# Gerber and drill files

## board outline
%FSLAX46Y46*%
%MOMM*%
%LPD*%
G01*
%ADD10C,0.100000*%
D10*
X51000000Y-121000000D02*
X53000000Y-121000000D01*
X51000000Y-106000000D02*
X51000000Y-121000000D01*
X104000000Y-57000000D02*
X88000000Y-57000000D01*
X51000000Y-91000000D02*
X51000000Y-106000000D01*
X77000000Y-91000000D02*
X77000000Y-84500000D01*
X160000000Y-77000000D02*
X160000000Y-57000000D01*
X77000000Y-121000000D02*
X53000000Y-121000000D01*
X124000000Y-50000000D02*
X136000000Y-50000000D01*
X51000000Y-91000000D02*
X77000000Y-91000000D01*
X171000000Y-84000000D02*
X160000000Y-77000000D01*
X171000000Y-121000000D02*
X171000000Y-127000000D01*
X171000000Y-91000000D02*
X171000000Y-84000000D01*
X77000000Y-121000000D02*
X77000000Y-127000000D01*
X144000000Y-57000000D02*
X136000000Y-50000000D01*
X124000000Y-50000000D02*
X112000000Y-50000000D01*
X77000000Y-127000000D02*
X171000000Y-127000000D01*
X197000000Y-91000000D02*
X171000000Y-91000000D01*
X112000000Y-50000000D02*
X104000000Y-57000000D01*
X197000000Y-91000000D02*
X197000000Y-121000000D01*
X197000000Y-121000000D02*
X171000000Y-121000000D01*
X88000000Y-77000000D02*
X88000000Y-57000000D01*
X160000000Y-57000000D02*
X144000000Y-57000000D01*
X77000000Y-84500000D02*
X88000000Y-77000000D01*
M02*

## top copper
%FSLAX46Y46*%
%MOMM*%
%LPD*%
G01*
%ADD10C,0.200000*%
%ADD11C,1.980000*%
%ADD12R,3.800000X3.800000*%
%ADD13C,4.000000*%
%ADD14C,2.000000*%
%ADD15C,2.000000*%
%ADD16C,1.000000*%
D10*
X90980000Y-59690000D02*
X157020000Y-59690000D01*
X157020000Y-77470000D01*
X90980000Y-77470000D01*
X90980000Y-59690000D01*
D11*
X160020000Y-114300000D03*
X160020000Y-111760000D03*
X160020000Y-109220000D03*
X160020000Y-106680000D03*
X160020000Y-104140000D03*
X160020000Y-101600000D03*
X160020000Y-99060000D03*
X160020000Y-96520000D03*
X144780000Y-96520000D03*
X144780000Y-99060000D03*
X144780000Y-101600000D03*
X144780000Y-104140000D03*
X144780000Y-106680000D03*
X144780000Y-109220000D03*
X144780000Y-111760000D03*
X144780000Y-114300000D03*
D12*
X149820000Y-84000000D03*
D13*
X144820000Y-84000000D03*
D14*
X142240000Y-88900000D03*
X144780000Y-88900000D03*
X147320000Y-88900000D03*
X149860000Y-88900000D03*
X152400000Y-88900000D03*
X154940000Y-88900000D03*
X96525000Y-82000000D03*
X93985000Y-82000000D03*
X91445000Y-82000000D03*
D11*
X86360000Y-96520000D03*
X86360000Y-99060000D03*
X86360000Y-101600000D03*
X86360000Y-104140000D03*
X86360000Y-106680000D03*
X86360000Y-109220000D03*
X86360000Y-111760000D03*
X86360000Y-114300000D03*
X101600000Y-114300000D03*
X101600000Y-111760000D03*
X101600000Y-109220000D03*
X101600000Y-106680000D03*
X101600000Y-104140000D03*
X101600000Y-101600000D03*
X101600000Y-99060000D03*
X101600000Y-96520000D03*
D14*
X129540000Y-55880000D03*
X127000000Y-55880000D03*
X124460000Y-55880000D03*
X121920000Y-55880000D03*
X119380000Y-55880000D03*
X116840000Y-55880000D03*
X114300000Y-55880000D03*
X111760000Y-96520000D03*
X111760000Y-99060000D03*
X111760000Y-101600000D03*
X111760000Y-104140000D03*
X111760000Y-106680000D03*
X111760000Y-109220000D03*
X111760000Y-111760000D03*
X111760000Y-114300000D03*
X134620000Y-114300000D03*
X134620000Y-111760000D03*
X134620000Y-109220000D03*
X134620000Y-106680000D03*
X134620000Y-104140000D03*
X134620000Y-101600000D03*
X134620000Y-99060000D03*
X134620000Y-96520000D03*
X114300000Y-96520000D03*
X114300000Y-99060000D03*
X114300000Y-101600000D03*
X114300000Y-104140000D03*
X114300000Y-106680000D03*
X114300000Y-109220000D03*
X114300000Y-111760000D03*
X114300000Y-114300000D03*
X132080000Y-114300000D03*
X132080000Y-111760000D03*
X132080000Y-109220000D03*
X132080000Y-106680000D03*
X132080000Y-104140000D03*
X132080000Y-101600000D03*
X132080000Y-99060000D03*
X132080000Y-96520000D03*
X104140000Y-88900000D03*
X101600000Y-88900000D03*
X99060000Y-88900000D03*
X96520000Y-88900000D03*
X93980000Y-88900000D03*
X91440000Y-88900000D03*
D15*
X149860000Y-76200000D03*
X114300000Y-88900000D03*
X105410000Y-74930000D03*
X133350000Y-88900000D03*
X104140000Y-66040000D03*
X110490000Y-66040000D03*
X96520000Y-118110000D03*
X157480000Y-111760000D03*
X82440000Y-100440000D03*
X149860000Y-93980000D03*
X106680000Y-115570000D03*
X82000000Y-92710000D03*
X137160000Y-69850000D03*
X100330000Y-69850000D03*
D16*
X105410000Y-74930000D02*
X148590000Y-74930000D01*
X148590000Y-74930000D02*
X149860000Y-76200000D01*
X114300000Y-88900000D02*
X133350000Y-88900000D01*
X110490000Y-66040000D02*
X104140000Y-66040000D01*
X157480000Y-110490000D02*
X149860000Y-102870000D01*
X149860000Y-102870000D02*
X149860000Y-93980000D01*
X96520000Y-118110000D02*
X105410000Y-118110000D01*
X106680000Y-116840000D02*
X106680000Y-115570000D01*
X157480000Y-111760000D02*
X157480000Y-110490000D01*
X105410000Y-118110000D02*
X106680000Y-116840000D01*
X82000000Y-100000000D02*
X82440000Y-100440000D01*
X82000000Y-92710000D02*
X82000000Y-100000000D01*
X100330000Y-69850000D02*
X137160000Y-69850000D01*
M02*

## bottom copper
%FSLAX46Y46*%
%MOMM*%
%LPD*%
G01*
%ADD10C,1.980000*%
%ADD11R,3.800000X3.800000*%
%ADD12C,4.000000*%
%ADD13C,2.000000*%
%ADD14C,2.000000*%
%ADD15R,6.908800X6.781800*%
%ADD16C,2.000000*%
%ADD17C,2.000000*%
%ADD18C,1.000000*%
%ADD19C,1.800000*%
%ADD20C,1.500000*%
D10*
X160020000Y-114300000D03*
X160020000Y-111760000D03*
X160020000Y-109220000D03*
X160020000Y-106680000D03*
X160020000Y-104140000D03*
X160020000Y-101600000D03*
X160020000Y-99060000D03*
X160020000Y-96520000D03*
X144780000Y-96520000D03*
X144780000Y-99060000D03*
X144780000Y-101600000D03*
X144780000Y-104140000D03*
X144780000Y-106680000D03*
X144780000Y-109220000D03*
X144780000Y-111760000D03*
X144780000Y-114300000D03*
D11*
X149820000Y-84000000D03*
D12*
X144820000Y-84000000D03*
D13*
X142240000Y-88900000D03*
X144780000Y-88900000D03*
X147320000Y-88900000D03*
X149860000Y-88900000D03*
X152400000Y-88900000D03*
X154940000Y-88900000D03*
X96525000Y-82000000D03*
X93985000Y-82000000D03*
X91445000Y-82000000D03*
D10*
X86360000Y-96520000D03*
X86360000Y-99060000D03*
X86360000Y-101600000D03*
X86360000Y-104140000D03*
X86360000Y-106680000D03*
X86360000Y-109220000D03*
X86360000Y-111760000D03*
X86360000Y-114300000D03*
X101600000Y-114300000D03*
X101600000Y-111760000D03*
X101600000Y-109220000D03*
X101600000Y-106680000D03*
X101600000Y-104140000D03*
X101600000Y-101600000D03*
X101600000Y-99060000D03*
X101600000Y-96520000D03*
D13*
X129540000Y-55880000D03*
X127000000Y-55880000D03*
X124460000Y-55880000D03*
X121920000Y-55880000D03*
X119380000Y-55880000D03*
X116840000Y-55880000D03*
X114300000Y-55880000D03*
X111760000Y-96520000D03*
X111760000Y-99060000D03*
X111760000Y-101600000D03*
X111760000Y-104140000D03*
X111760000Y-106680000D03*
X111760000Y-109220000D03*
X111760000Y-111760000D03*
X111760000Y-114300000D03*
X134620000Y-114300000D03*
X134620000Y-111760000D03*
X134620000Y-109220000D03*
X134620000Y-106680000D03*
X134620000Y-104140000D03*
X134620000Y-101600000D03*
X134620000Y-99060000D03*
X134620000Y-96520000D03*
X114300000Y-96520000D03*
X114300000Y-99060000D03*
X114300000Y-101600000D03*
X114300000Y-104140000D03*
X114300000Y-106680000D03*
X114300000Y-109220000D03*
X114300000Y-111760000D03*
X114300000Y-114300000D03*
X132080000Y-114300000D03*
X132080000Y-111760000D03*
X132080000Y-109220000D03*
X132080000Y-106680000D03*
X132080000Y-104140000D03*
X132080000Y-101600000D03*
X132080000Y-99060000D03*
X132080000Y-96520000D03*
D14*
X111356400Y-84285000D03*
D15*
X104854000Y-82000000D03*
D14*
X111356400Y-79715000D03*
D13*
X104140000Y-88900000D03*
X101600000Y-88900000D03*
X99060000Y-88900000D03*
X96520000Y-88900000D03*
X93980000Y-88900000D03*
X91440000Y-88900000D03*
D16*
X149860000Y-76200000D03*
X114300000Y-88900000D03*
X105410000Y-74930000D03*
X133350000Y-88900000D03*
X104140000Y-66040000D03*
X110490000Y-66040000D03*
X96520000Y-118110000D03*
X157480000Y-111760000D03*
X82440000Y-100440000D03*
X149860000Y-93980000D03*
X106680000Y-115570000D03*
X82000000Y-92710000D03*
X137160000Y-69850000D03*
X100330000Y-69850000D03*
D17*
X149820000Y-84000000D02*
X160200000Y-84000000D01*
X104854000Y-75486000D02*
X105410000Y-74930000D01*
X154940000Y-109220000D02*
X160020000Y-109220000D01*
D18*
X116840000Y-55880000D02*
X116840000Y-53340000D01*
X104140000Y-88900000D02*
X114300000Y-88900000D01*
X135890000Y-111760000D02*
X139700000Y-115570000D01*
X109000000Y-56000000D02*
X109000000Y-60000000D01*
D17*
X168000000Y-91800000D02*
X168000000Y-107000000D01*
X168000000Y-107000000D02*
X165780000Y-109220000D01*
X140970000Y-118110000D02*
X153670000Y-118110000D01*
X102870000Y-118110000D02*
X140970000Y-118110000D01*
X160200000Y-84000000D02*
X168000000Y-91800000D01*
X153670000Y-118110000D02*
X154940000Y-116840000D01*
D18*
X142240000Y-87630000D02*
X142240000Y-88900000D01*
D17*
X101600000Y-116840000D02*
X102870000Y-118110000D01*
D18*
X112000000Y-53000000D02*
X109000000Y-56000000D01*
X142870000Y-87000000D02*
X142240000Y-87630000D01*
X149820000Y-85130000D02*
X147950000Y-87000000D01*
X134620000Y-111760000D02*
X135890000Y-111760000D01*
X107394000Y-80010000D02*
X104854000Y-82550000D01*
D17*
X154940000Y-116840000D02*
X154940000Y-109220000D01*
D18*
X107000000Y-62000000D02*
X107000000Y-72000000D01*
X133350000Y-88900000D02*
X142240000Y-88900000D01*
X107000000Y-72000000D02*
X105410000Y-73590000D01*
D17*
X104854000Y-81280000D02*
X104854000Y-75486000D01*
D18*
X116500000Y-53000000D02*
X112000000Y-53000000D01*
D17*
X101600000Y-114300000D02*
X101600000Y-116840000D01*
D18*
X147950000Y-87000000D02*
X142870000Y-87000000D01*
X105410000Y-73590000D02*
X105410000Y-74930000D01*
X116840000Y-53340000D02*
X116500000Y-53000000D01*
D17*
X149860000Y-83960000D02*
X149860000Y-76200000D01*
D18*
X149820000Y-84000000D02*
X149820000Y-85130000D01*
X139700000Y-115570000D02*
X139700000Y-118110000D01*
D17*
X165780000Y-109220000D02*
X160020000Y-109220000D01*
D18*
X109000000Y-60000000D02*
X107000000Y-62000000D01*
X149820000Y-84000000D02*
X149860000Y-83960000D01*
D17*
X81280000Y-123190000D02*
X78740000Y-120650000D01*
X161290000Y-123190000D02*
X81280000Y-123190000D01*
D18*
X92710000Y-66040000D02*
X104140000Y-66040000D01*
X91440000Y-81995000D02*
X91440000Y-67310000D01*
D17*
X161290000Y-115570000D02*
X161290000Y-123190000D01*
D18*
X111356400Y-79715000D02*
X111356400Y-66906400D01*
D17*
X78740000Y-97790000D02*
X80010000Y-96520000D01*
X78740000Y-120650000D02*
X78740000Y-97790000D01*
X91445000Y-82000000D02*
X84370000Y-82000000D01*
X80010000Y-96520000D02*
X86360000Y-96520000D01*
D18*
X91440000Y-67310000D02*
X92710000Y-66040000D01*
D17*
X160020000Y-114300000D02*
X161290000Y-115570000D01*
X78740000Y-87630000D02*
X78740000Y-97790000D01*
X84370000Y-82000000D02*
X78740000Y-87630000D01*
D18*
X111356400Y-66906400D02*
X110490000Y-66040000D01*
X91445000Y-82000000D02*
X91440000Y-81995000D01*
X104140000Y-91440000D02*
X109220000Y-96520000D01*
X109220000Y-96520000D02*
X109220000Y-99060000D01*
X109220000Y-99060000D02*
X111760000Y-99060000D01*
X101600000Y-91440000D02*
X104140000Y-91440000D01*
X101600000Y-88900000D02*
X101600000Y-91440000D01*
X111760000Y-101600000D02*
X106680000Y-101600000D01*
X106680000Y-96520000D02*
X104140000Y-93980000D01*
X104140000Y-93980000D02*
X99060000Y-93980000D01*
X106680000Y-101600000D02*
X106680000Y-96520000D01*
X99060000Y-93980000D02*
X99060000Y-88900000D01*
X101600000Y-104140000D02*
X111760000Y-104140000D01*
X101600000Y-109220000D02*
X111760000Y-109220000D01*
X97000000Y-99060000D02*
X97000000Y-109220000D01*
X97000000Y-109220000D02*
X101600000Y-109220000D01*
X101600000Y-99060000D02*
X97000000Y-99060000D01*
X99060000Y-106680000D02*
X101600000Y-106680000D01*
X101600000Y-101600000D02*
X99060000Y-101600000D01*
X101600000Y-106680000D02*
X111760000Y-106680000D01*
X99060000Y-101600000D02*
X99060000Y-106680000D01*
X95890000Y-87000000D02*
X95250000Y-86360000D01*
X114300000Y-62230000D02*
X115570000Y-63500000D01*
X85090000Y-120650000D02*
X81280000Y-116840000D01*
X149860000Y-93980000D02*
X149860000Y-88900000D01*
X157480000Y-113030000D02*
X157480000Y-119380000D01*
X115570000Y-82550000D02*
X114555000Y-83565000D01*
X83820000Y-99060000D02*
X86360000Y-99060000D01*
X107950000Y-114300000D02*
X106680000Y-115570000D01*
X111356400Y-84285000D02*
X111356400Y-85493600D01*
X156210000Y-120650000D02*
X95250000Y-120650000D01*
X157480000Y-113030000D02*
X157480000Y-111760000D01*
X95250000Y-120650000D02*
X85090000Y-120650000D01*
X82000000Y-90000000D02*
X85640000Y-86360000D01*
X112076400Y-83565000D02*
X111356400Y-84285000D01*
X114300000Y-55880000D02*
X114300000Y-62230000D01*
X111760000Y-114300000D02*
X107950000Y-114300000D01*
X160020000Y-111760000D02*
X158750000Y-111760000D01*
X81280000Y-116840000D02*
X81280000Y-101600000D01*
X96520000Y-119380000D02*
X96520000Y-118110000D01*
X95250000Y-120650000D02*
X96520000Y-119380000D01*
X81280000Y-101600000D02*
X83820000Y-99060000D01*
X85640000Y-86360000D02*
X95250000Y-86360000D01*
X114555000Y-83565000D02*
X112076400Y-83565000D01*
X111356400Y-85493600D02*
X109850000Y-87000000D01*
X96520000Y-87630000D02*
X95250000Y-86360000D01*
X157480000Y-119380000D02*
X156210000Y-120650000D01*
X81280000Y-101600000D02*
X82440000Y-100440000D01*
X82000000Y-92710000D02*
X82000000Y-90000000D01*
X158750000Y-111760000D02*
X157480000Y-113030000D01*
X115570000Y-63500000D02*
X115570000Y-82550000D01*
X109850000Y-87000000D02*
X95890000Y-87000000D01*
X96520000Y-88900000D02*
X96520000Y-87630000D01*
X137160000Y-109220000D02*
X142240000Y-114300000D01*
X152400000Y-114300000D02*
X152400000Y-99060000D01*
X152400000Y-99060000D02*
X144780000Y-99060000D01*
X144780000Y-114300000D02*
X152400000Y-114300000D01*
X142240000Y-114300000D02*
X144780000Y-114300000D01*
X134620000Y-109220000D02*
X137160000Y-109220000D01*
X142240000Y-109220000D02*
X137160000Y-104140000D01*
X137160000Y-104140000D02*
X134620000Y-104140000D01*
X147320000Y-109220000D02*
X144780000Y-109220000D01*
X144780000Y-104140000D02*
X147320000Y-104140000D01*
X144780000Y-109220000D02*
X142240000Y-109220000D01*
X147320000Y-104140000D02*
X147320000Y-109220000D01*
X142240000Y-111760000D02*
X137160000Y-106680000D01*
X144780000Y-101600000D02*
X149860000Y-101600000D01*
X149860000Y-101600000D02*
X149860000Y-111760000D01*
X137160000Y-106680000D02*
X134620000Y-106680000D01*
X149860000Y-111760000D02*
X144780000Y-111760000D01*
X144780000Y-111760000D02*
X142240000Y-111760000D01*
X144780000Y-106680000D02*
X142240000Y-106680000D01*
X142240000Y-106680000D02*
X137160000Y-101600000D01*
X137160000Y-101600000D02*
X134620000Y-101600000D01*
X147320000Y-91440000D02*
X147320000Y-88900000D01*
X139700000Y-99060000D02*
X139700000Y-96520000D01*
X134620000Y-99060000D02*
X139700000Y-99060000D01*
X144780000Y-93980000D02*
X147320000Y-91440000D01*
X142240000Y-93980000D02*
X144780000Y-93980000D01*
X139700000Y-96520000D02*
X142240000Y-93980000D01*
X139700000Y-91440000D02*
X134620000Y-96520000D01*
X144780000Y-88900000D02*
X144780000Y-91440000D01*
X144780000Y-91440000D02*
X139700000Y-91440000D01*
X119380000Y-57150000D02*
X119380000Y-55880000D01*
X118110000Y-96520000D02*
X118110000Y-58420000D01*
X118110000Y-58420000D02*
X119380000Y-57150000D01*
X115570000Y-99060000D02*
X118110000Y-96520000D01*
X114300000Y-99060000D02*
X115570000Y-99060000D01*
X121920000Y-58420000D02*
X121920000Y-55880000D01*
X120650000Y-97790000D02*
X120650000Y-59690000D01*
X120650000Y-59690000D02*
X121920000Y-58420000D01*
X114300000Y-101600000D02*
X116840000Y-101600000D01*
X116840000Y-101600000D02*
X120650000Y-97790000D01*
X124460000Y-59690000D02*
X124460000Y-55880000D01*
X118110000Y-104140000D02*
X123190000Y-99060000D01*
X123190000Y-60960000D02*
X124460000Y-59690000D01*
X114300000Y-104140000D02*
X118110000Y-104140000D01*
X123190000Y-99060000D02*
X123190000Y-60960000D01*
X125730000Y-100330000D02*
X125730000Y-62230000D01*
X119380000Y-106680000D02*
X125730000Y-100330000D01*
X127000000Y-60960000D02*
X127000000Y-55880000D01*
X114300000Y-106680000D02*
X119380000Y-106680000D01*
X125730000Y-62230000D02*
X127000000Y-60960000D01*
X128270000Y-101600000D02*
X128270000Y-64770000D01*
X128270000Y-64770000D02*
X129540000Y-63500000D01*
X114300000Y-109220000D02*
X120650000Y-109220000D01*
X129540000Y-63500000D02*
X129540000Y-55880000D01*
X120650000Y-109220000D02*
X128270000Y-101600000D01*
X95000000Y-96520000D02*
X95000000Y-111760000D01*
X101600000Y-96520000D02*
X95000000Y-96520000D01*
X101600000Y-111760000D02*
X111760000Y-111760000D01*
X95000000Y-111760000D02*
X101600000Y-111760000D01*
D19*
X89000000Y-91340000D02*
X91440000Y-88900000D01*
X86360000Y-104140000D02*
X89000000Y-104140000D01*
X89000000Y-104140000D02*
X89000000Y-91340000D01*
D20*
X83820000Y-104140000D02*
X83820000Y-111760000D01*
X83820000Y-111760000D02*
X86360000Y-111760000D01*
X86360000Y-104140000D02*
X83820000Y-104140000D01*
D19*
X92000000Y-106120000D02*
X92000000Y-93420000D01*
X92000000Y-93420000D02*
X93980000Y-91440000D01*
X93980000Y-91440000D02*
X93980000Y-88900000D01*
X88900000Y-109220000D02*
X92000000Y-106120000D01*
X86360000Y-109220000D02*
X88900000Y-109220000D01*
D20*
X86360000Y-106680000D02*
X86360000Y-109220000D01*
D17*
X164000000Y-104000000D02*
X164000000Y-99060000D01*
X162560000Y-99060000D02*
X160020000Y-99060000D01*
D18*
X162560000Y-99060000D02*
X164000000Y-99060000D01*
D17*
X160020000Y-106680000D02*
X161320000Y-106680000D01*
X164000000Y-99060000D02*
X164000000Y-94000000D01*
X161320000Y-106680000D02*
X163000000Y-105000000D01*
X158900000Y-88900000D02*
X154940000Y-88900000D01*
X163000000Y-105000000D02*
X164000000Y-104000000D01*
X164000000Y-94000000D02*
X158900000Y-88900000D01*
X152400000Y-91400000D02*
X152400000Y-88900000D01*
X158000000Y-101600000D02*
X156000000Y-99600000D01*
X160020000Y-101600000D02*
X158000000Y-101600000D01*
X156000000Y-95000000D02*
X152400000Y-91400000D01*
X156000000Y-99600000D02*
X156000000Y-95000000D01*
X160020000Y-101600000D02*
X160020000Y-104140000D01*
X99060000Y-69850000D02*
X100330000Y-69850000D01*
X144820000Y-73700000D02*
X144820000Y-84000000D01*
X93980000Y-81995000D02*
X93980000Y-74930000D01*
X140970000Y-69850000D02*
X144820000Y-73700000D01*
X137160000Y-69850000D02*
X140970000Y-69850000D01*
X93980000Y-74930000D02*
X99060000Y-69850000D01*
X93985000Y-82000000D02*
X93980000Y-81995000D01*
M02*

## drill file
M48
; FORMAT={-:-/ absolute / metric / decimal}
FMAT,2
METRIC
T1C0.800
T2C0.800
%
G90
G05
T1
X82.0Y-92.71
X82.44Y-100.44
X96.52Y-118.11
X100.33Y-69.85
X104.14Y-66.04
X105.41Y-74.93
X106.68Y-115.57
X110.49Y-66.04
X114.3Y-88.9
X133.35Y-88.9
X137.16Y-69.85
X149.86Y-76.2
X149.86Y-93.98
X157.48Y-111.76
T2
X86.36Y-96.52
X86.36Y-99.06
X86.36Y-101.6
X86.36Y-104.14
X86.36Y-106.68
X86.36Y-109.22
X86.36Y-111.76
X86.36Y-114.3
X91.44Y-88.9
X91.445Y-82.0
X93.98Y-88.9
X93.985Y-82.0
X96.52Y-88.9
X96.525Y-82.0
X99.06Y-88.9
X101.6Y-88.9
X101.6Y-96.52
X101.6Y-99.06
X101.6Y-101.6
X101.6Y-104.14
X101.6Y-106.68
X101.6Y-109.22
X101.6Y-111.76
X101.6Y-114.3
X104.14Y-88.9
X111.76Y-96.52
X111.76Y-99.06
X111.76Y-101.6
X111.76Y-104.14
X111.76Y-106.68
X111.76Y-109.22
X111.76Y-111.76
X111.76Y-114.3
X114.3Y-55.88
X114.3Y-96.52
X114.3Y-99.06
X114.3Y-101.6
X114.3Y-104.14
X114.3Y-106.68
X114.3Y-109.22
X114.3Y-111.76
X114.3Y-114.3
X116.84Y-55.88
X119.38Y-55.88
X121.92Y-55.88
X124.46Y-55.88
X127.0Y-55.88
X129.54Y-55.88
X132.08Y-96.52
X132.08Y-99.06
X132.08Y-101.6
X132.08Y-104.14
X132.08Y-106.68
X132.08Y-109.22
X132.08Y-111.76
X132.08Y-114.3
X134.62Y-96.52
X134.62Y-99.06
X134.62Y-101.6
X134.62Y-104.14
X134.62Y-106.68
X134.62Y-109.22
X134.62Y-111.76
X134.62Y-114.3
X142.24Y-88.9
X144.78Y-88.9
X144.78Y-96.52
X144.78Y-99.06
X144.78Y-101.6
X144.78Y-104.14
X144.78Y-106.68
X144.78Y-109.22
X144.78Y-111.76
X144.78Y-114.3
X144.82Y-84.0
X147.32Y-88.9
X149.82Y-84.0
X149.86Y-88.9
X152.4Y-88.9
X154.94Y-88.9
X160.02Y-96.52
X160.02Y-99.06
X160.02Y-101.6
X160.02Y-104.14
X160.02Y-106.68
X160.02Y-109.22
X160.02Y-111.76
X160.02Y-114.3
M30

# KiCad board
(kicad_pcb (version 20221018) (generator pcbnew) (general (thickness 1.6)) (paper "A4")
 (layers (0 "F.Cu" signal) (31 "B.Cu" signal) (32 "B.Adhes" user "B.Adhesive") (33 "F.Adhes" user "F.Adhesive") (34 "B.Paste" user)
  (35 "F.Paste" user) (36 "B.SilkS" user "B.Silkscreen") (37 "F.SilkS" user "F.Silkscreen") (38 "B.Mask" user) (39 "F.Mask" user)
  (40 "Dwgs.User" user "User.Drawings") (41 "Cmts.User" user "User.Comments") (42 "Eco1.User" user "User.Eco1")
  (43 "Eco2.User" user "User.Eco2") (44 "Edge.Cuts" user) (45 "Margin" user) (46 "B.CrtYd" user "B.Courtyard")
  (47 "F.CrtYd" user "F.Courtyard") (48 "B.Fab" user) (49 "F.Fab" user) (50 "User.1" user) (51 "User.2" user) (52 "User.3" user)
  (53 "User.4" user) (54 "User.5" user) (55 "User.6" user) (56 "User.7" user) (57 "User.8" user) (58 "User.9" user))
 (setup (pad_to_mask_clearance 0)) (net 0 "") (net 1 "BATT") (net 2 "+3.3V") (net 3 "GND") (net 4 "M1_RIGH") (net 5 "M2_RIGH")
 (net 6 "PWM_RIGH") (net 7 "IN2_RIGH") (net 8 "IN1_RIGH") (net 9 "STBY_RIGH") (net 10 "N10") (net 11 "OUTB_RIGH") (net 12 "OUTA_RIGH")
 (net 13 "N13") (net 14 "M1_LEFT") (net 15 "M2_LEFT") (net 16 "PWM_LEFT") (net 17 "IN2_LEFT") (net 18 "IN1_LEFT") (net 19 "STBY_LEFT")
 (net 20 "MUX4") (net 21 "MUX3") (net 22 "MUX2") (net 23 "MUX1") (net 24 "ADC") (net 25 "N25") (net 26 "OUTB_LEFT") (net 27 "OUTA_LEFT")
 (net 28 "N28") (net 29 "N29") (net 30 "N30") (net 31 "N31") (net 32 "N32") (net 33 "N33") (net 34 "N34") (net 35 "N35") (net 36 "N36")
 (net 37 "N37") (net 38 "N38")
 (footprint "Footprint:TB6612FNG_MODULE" (layer "F.Cu") (at 152.4 105.41 180)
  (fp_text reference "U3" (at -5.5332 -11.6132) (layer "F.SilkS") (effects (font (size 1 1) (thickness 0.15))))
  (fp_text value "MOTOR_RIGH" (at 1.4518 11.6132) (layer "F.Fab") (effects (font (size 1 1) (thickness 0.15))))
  (pad "1" thru_hole circle (at -7.62 -8.89 180) (size 1.98 1.98) (drill 0.8) (layers "*.Cu" "*.Mask") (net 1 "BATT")
   (solder_mask_margin 0.102))
  (pad "2" thru_hole circle (at -7.62 -6.35 180) (size 1.98 1.98) (drill 0.8) (layers "*.Cu" "*.Mask") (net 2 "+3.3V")
   (solder_mask_margin 0.102))
  (pad "3" thru_hole circle (at -7.62 -3.81 180) (size 1.98 1.98) (drill 0.8) (layers "*.Cu" "*.Mask") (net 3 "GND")
   (solder_mask_margin 0.102))
  (pad "4" thru_hole circle (at -7.62 -1.27 180) (size 1.98 1.98) (drill 0.8) (layers "*.Cu" "*.Mask") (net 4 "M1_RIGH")
   (solder_mask_margin 0.102))
  (pad "5" thru_hole circle (at -7.62 1.27 180) (size 1.98 1.98) (drill 0.8) (layers "*.Cu" "*.Mask") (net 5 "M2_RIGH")
   (solder_mask_margin 0.102))
  (pad "6" thru_hole circle (at -7.62 3.81 180) (size 1.98 1.98) (drill 0.8) (layers "*.Cu" "*.Mask") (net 5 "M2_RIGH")
   (solder_mask_margin 0.102))
  (pad "7" thru_hole circle (at -7.62 6.35 180) (size 1.98 1.98) (drill 0.8) (layers "*.Cu" "*.Mask") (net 4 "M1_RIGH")
   (solder_mask_margin 0.102))
  (pad "8" thru_hole circle (at -7.62 8.89 180) (size 1.98 1.98) (drill 0.8) (layers "*.Cu" "*.Mask") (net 3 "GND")
   (solder_mask_margin 0.102))
  (pad "9" thru_hole circle (at 7.62 8.89 180) (size 1.98 1.98) (drill 0.8) (layers "*.Cu" "*.Mask") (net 3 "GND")
   (solder_mask_margin 0.102))
  (pad "10" thru_hole circle (at 7.62 6.35 180) (size 1.98 1.98) (drill 0.8) (layers "*.Cu" "*.Mask") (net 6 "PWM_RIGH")
   (solder_mask_margin 0.102))
  (pad "11" thru_hole circle (at 7.62 3.81 180) (size 1.98 1.98) (drill 0.8) (layers "*.Cu" "*.Mask") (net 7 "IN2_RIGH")
   (solder_mask_margin 0.102))
  (pad "12" thru_hole circle (at 7.62 1.27 180) (size 1.98 1.98) (drill 0.8) (layers "*.Cu" "*.Mask") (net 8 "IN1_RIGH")
   (solder_mask_margin 0.102))
  (pad "13" thru_hole circle (at 7.62 -1.27 180) (size 1.98 1.98) (drill 0.8) (layers "*.Cu" "*.Mask") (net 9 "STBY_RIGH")
   (solder_mask_margin 0.102))
  (pad "14" thru_hole circle (at 7.62 -3.81 180) (size 1.98 1.98) (drill 0.8) (layers "*.Cu" "*.Mask") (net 8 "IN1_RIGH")
   (solder_mask_margin 0.102))
  (pad "15" thru_hole circle (at 7.62 -6.35 180) (size 1.98 1.98) (drill 0.8) (layers "*.Cu" "*.Mask") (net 7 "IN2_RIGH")
   (solder_mask_margin 0.102))
  (pad "16" thru_hole circle (at 7.62 -8.89 180) (size 1.98 1.98) (drill 0.8) (layers "*.Cu" "*.Mask") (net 6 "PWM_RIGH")
   (solder_mask_margin 0.102)))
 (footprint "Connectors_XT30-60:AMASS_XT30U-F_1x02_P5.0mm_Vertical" (layer "F.Cu") (at 149.82 84 180)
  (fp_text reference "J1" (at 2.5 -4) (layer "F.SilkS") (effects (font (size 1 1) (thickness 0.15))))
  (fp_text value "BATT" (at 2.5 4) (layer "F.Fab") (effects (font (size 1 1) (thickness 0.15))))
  (pad "1" thru_hole rect (at 0 0 180) (size 3.8 3.8) (drill 0.8) (layers "*.Cu" "*.Mask") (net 3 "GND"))
  (pad "2" thru_hole circle (at 5 0 180) (size 4 4) (drill 0.8) (layers "*.Cu" "*.Mask") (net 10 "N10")))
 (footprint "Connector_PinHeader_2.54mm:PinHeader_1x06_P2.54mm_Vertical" (layer "F.Cu") (at 142.24 88.9 90)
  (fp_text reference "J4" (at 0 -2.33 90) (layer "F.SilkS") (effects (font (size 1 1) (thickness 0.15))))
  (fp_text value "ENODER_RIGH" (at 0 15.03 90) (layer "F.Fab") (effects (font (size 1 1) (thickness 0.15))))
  (pad "1" thru_hole circle (at 0 0 90) (size 2 2) (drill 0.8) (layers "*.Cu" "*.Mask") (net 3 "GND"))
  (pad "2" thru_hole circle (at 0 2.54 90) (size 2 2) (drill 0.8) (layers "*.Cu" "*.Mask") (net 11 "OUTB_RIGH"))
  (pad "3" thru_hole circle (at 0 5.08 90) (size 2 2) (drill 0.8) (layers "*.Cu" "*.Mask") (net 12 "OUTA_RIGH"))
  (pad "4" thru_hole circle (at 0 7.62 90) (size 2 2) (drill 0.8) (layers "*.Cu" "*.Mask") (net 2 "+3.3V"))
  (pad "5" thru_hole circle (at 0 10.16 90) (size 2 2) (drill 0.8) (layers "*.Cu" "*.Mask") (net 5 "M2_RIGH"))
  (pad "6" thru_hole circle (at 0 12.7 90) (size 2 2) (drill 0.8) (layers "*.Cu" "*.Mask") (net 4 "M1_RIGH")))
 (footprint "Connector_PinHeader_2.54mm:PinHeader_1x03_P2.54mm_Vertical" (layer "F.Cu") (at 96.525 82 -90)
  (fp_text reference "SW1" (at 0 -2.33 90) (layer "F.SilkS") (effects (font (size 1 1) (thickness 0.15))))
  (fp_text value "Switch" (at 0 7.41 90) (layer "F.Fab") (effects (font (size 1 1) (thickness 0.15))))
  (pad "1" thru_hole circle (at 0 0 270) (size 2 2) (drill 0.8) (layers "*.Cu" "*.Mask") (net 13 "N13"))
  (pad "2" thru_hole circle (at 0 2.54 270) (size 2 2) (drill 0.8) (layers "*.Cu" "*.Mask") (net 10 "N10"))
  (pad "3" thru_hole circle (at 0 5.08 270) (size 2 2) (drill 0.8) (layers "*.Cu" "*.Mask") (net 1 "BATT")))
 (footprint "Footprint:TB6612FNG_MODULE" (layer "F.Cu") (at 93.98 105.41)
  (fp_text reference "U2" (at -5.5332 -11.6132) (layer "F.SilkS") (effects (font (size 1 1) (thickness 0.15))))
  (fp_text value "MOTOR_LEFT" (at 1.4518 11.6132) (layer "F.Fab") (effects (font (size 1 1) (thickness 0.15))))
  (pad "1" thru_hole circle (at -7.62 -8.89) (size 1.98 1.98) (drill 0.8) (layers "*.Cu" "*.Mask") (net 1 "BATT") (solder_mask_margin 0.102))
  (pad "2" thru_hole circle (at -7.62 -6.35) (size 1.98 1.98) (drill 0.8) (layers "*.Cu" "*.Mask") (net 2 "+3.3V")
   (solder_mask_margin 0.102))
  (pad "3" thru_hole circle (at -7.62 -3.81) (size 1.98 1.98) (drill 0.8) (layers "*.Cu" "*.Mask") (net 3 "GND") (solder_mask_margin 0.102))
  (pad "4" thru_hole circle (at -7.62 -1.27) (size 1.98 1.98) (drill 0.8) (layers "*.Cu" "*.Mask") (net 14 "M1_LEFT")
   (solder_mask_margin 0.102))
  (pad "5" thru_hole circle (at -7.62 1.27) (size 1.98 1.98) (drill 0.8) (layers "*.Cu" "*.Mask") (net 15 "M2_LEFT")
   (solder_mask_margin 0.102))
  (pad "6" thru_hole circle (at -7.62 3.81) (size 1.98 1.98) (drill 0.8) (layers "*.Cu" "*.Mask") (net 15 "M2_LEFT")
   (solder_mask_margin 0.102))
  (pad "7" thru_hole circle (at -7.62 6.35) (size 1.98 1.98) (drill 0.8) (layers "*.Cu" "*.Mask") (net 14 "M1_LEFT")
   (solder_mask_margin 0.102))
  (pad "8" thru_hole circle (at -7.62 8.89) (size 1.98 1.98) (drill 0.8) (layers "*.Cu" "*.Mask") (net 3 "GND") (solder_mask_margin 0.102))
  (pad "9" thru_hole circle (at 7.62 8.89) (size 1.98 1.98) (drill 0.8) (layers "*.Cu" "*.Mask") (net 3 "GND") (solder_mask_margin 0.102))
  (pad "10" thru_hole circle (at 7.62 6.35) (size 1.98 1.98) (drill 0.8) (layers "*.Cu" "*.Mask") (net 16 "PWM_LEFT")
   (solder_mask_margin 0.102))
  (pad "11" thru_hole circle (at 7.62 3.81) (size 1.98 1.98) (drill 0.8) (layers "*.Cu" "*.Mask") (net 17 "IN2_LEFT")
   (solder_mask_margin 0.102))
  (pad "12" thru_hole circle (at 7.62 1.27) (size 1.98 1.98) (drill 0.8) (layers "*.Cu" "*.Mask") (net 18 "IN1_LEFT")
   (solder_mask_margin 0.102))
  (pad "13" thru_hole circle (at 7.62 -1.27) (size 1.98 1.98) (drill 0.8) (layers "*.Cu" "*.Mask") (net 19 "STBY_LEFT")
   (solder_mask_margin 0.102))
  (pad "14" thru_hole circle (at 7.62 -3.81) (size 1.98 1.98) (drill 0.8) (layers "*.Cu" "*.Mask") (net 18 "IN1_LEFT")
   (solder_mask_margin 0.102))
  (pad "15" thru_hole circle (at 7.62 -6.35) (size 1.98 1.98) (drill 0.8) (layers "*.Cu" "*.Mask") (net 17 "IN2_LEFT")
   (solder_mask_margin 0.102))
  (pad "16" thru_hole circle (at 7.62 -8.89) (size 1.98 1.98) (drill 0.8) (layers "*.Cu" "*.Mask") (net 16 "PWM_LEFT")
   (solder_mask_margin 0.102)))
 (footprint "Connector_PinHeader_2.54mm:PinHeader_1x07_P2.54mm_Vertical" (layer "F.Cu") (at 129.54 55.88 -90)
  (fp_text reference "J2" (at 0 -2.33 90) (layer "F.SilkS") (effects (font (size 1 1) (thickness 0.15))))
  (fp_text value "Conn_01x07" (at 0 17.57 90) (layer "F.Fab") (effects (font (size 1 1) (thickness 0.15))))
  (pad "1" thru_hole circle (at 0 0 270) (size 2 2) (drill 0.8) (layers "*.Cu" "*.Mask") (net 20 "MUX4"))
  (pad "2" thru_hole circle (at 0 2.54 270) (size 2 2) (drill 0.8) (layers "*.Cu" "*.Mask") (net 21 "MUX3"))
  (pad "3" thru_hole circle (at 0 5.08 270) (size 2 2) (drill 0.8) (layers "*.Cu" "*.Mask") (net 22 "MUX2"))
  (pad "4" thru_hole circle (at 0 7.62 270) (size 2 2) (drill 0.8) (layers "*.Cu" "*.Mask") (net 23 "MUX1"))
  (pad "5" thru_hole circle (at 0 10.16 270) (size 2 2) (drill 0.8) (layers "*.Cu" "*.Mask") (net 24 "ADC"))
  (pad "6" thru_hole circle (at 0 12.7 270) (size 2 2) (drill 0.8) (layers "*.Cu" "*.Mask") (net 3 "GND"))
  (pad "7" thru_hole circle (at 0 15.24 270) (size 2 2) (drill 0.8) (layers "*.Cu" "*.Mask") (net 2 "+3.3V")))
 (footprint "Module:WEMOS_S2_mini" (layer "F.Cu") (at 111.76 96.52)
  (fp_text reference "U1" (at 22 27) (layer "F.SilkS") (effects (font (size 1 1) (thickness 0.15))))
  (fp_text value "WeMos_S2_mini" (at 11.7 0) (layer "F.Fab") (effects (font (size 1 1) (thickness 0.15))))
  (pad "1" thru_hole circle (at 0 0) (size 2 2) (drill 0.8) (layers "*.Cu" "*.Mask") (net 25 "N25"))
  (pad "2" thru_hole circle (at 0 2.54) (size 2 2) (drill 0.8) (layers "*.Cu" "*.Mask") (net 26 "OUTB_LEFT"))
  (pad "3" thru_hole circle (at 0 5.08) (size 2 2) (drill 0.8) (layers "*.Cu" "*.Mask") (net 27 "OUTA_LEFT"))
  (pad "4" thru_hole circle (at 0 7.62) (size 2 2) (drill 0.8) (layers "*.Cu" "*.Mask") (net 19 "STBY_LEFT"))
  (pad "5" thru_hole circle (at 0 10.16) (size 2 2) (drill 0.8) (layers "*.Cu" "*.Mask") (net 18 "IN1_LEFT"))
  (pad "6" thru_hole circle (at 0 12.7) (size 2 2) (drill 0.8) (layers "*.Cu" "*.Mask") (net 17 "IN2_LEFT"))
  (pad "7" thru_hole circle (at 0 15.24) (size 2 2) (drill 0.8) (layers "*.Cu" "*.Mask") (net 16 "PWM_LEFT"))
  (pad "8" thru_hole circle (at 0 17.78) (size 2 2) (drill 0.8) (layers "*.Cu" "*.Mask") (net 2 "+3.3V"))
  (pad "9" thru_hole circle (at 22.86 17.78) (size 2 2) (drill 0.8) (layers "*.Cu" "*.Mask") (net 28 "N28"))
  (pad "10" thru_hole circle (at 22.86 15.24) (size 2 2) (drill 0.8) (layers "*.Cu" "*.Mask") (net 3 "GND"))
  (pad "11" thru_hole circle (at 22.86 12.7) (size 2 2) (drill 0.8) (layers "*.Cu" "*.Mask") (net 6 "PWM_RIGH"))
  (pad "12" thru_hole circle (at 22.86 10.16) (size 2 2) (drill 0.8) (layers "*.Cu" "*.Mask") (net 7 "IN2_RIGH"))
  (pad "13" thru_hole circle (at 22.86 7.62) (size 2 2) (drill 0.8) (layers "*.Cu" "*.Mask") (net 8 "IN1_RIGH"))
  (pad "14" thru_hole circle (at 22.86 5.08) (size 2 2) (drill 0.8) (layers "*.Cu" "*.Mask") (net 9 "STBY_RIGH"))
  (pad "15" thru_hole circle (at 22.86 2.54) (size 2 2) (drill 0.8) (layers "*.Cu" "*.Mask") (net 12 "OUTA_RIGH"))
  (pad "16" thru_hole circle (at 22.86 0) (size 2 2) (drill 0.8) (layers "*.Cu" "*.Mask") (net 11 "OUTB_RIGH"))
  (pad "17" thru_hole circle (at 2.54 0) (size 2 2) (drill 0.8) (layers "*.Cu" "*.Mask") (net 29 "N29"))
  (pad "18" thru_hole circle (at 2.54 2.54) (size 2 2) (drill 0.8) (layers "*.Cu" "*.Mask") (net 24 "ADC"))
  (pad "19" thru_hole circle (at 2.54 5.08) (size 2 2) (drill 0.8) (layers "*.Cu" "*.Mask") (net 23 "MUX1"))
  (pad "20" thru_hole circle (at 2.54 7.62) (size 2 2) (drill 0.8) (layers "*.Cu" "*.Mask") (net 22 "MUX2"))
  (pad "21" thru_hole circle (at 2.54 10.16) (size 2 2) (drill 0.8) (layers "*.Cu" "*.Mask") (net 21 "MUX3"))
  (pad "22" thru_hole circle (at 2.54 12.7) (size 2 2) (drill 0.8) (layers "*.Cu" "*.Mask") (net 20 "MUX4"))
  (pad "23" thru_hole circle (at 2.54 15.24) (size 2 2) (drill 0.8) (layers "*.Cu" "*.Mask") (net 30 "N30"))
  (pad "24" thru_hole circle (at 2.54 17.78) (size 2 2) (drill 0.8) (layers "*.Cu" "*.Mask") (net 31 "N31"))
  (pad "25" thru_hole circle (at 20.32 17.78) (size 2 2) (drill 0.8) (layers "*.Cu" "*.Mask") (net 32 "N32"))
  (pad "26" thru_hole circle (at 20.32 15.24) (size 2 2) (drill 0.8) (layers "*.Cu" "*.Mask") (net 3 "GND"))
  (pad "27" thru_hole circle (at 20.32 12.7) (size 2 2) (drill 0.8) (layers "*.Cu" "*.Mask") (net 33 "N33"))
  (pad "28" thru_hole circle (at 20.32 10.16) (size 2 2) (drill 0.8) (layers "*.Cu" "*.Mask") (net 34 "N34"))
  (pad "29" thru_hole circle (at 20.32 7.62) (size 2 2) (drill 0.8) (layers "*.Cu" "*.Mask") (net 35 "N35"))
  (pad "30" thru_hole circle (at 20.32 5.08) (size 2 2) (drill 0.8) (layers "*.Cu" "*.Mask") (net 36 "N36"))
  (pad "31" thru_hole circle (at 20.32 2.54) (size 2 2) (drill 0.8) (layers "*.Cu" "*.Mask") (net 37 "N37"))
  (pad "32" thru_hole circle (at 20.32 0) (size 2 2) (drill 0.8) (layers "*.Cu" "*.Mask") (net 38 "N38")))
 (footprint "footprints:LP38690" (layer "F.Cu") (at 104.854 82 90)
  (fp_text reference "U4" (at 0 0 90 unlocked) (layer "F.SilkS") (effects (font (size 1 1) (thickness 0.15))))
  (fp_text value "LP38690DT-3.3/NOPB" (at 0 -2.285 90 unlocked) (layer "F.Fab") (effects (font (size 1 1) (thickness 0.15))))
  (pad "1" smd circle (at -2.285 6.5024 90) (size 2 2) (layers "B.Cu" "F.Paste" "F.Mask") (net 2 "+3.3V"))
  (pad "2" smd rect (at 0 0 90) (size 6.7818 6.9088) (layers "B.Cu" "F.Paste" "F.Mask") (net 3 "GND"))
  (pad "3" smd circle (at 2.285 6.5024 90) (size 2 2) (layers "B.Cu" "F.Paste" "F.Mask") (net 1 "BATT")))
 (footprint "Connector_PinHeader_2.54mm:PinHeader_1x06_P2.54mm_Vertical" (layer "F.Cu") (at 104.14 88.9 -90)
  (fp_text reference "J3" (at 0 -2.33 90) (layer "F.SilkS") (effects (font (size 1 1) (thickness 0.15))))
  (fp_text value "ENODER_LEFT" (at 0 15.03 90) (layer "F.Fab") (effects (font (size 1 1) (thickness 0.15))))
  (pad "1" thru_hole circle (at 0 0 270) (size 2 2) (drill 0.8) (layers "*.Cu" "*.Mask") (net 3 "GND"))
  (pad "2" thru_hole circle (at 0 2.54 270) (size 2 2) (drill 0.8) (layers "*.Cu" "*.Mask") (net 26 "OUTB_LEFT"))
  (pad "3" thru_hole circle (at 0 5.08 270) (size 2 2) (drill 0.8) (layers "*.Cu" "*.Mask") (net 27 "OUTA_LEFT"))
  (pad "4" thru_hole circle (at 0 7.62 270) (size 2 2) (drill 0.8) (layers "*.Cu" "*.Mask") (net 2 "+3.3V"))
  (pad "5" thru_hole circle (at 0 10.16 270) (size 2 2) (drill 0.8) (layers "*.Cu" "*.Mask") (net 15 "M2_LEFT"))
  (pad "6" thru_hole circle (at 0 12.7 270) (size 2 2) (drill 0.8) (layers "*.Cu" "*.Mask") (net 14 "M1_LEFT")))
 (gr_rect (start 90.98 59.69) (end 157.02 77.47) (stroke (width 0.2) (type default)) (fill none) (layer "F.Cu"))
 (gr_line (start 51 121) (end 53 121) (stroke (width 0.1) (type default)) (layer "Edge.Cuts"))
 (gr_line (start 51 106) (end 51 121) (stroke (width 0.1) (type default)) (layer "Edge.Cuts"))
 (gr_line (start 104 57) (end 88 57) (stroke (width 0.1) (type default)) (layer "Edge.Cuts"))
 (gr_line (start 51 91) (end 51 106) (stroke (width 0.1) (type default)) (layer "Edge.Cuts"))
 (gr_line (start 77 91) (end 77 84.5) (stroke (width 0.1) (type default)) (layer "Edge.Cuts"))
 (gr_line (start 160 77) (end 160 57) (stroke (width 0.1) (type default)) (layer "Edge.Cuts"))
 (gr_line (start 77 121) (end 53 121) (stroke (width 0.1) (type default)) (layer "Edge.Cuts"))
 (gr_line (start 124 50) (end 136 50) (stroke (width 0.1) (type default)) (layer "Edge.Cuts"))
 (gr_line (start 51 91) (end 77 91) (stroke (width 0.1) (type default)) (layer "Edge.Cuts"))
 (gr_line (start 171 84) (end 160 77) (stroke (width 0.1) (type default)) (layer "Edge.Cuts"))
 (gr_line (start 171 121) (end 171 127) (stroke (width 0.1) (type default)) (layer "Edge.Cuts"))
 (gr_line (start 171 91) (end 171 84) (stroke (width 0.1) (type default)) (layer "Edge.Cuts"))
 (gr_line (start 77 121) (end 77 127) (stroke (width 0.1) (type default)) (layer "Edge.Cuts"))
 (gr_line (start 144 57) (end 136 50) (stroke (width 0.1) (type default)) (layer "Edge.Cuts"))
 (gr_line (start 124 50) (end 112 50) (stroke (width 0.1) (type default)) (layer "Edge.Cuts"))
 (gr_line (start 77 127) (end 171 127) (stroke (width 0.1) (type default)) (layer "Edge.Cuts"))
 (gr_line (start 197 91) (end 171 91) (stroke (width 0.1) (type default)) (layer "Edge.Cuts"))
 (gr_line (start 112 50) (end 104 57) (stroke (width 0.1) (type default)) (layer "Edge.Cuts"))
 (gr_line (start 197 91) (end 197 121) (stroke (width 0.1) (type default)) (layer "Edge.Cuts"))
 (gr_line (start 197 121) (end 171 121) (stroke (width 0.1) (type default)) (layer "Edge.Cuts"))
 (gr_line (start 88 77) (end 88 57) (stroke (width 0.1) (type default)) (layer "Edge.Cuts"))
 (gr_line (start 160 57) (end 144 57) (stroke (width 0.1) (type default)) (layer "Edge.Cuts"))
 (gr_line (start 77 84.5) (end 88 77) (stroke (width 0.1) (type default)) (layer "Edge.Cuts"))
 (segment (start 105.41 74.93) (end 148.59 74.93) (width 1) (layer "F.Cu") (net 3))
 (segment (start 148.59 74.93) (end 149.86 76.2) (width 1) (layer "F.Cu") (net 3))
 (segment (start 114.3 88.9) (end 133.35 88.9) (width 1) (layer "F.Cu") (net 3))
 (via (at 149.86 76.2) (size 2) (drill 0.8) (layers "F.Cu" "B.Cu") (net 3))
 (via (at 114.3 88.9) (size 2) (drill 0.8) (layers "F.Cu" "B.Cu") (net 3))
 (via (at 105.41 74.93) (size 2) (drill 0.8) (layers "F.Cu" "B.Cu") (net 3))
 (via (at 133.35 88.9) (size 2) (drill 0.8) (layers "F.Cu" "B.Cu") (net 3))
 (segment (start 149.82 84) (end 160.2 84) (width 2) (layer "B.Cu") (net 3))
 (segment (start 104.854 75.486) (end 105.41 74.93) (width 2) (layer "B.Cu") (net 3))
 (segment (start 154.94 109.22) (end 160.02 109.22) (width 2) (layer "B.Cu") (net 3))
 (segment (start 116.84 55.88) (end 116.84 53.34) (width 1) (layer "B.Cu") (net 3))
 (segment (start 104.14 88.9) (end 114.3 88.9) (width 1) (layer "B.Cu") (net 3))
 (segment (start 135.89 111.76) (end 139.7 115.57) (width 1) (layer "B.Cu") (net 3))
 (segment (start 109 56) (end 109 60) (width 1) (layer "B.Cu") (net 3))
 (segment (start 168 91.8) (end 168 107) (width 2) (layer "B.Cu") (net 3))
 (segment (start 168 107) (end 165.78 109.22) (width 2) (layer "B.Cu") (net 3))
 (segment (start 140.97 118.11) (end 153.67 118.11) (width 2) (layer "B.Cu") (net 3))
 (segment (start 102.87 118.11) (end 140.97 118.11) (width 2) (layer "B.Cu") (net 3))
 (segment (start 160.2 84) (end 168 91.8) (width 2) (layer "B.Cu") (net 3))
 (segment (start 153.67 118.11) (end 154.94 116.84) (width 2) (layer "B.Cu") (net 3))
 (segment (start 142.24 87.63) (end 142.24 88.9) (width 1) (layer "B.Cu") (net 3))
 (segment (start 101.6 116.84) (end 102.87 118.11) (width 2) (layer "B.Cu") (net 3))
 (segment (start 112 53) (end 109 56) (width 1) (layer "B.Cu") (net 3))
 (segment (start 142.87 87) (end 142.24 87.63) (width 1) (layer "B.Cu") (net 3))
 (segment (start 149.82 85.13) (end 147.95 87) (width 1) (layer "B.Cu") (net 3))
 (segment (start 134.62 111.76) (end 135.89 111.76) (width 1) (layer "B.Cu") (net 3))
 (segment (start 107.394 80.01) (end 104.854 82.55) (width 1) (layer "B.Cu") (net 3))
 (segment (start 154.94 116.84) (end 154.94 109.22) (width 2) (layer "B.Cu") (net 3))
 (segment (start 107 62) (end 107 72) (width 1) (layer "B.Cu") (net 3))
 (segment (start 133.35 88.9) (end 142.24 88.9) (width 1) (layer "B.Cu") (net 3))
 (segment (start 107 72) (end 105.41 73.59) (width 1) (layer "B.Cu") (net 3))
 (segment (start 104.854 81.28) (end 104.854 75.486) (width 2) (layer "B.Cu") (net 3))
 (segment (start 116.5 53) (end 112 53) (width 1) (layer "B.Cu") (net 3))
 (segment (start 101.6 114.3) (end 101.6 116.84) (width 2) (layer "B.Cu") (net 3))
 (segment (start 147.95 87) (end 142.87 87) (width 1) (layer "B.Cu") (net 3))
 (segment (start 105.41 73.59) (end 105.41 74.93) (width 1) (layer "B.Cu") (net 3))
 (segment (start 116.84 53.34) (end 116.5 53) (width 1) (layer "B.Cu") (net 3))
 (segment (start 149.86 83.96) (end 149.86 76.2) (width 2) (layer "B.Cu") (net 3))
 (segment (start 149.82 84) (end 149.82 85.13) (width 1) (layer "B.Cu") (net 3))
 (segment (start 139.7 115.57) (end 139.7 118.11) (width 1) (layer "B.Cu") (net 3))
 (segment (start 165.78 109.22) (end 160.02 109.22) (width 2) (layer "B.Cu") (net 3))
 (segment (start 109 60) (end 107 62) (width 1) (layer "B.Cu") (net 3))
 (segment (start 149.82 84) (end 149.86 83.96) (width 1) (layer "B.Cu") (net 3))
 (segment (start 110.49 66.04) (end 104.14 66.04) (width 1) (layer "F.Cu") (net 1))
 (via (at 104.14 66.04) (size 2) (drill 0.8) (layers "F.Cu" "B.Cu") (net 1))
 (via (at 110.49 66.04) (size 2) (drill 0.8) (layers "F.Cu" "B.Cu") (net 1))
 (segment (start 81.28 123.19) (end 78.74 120.65) (width 2) (layer "B.Cu") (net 1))
 (segment (start 161.29 123.19) (end 81.28 123.19) (width 2) (layer "B.Cu") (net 1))
 (segment (start 92.71 66.04) (end 104.14 66.04) (width 1) (layer "B.Cu") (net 1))
 (segment (start 91.44 81.995) (end 91.44 67.31) (width 1) (layer "B.Cu") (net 1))
 (segment (start 161.29 115.57) (end 161.29 123.19) (width 2) (layer "B.Cu") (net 1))
 (segment (start 111.3564 79.715) (end 111.3564 66.9064) (width 1) (layer "B.Cu") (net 1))
 (segment (start 78.74 97.79) (end 80.01 96.52) (width 2) (layer "B.Cu") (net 1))
 (segment (start 78.74 120.65) (end 78.74 97.79) (width 2) (layer "B.Cu") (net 1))
 (segment (start 91.445 82) (end 84.37 82) (width 2) (layer "B.Cu") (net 1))
 (segment (start 80.01 96.52) (end 86.36 96.52) (width 2) (layer "B.Cu") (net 1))
 (segment (start 91.44 67.31) (end 92.71 66.04) (width 1) (layer "B.Cu") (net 1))
 (segment (start 160.02 114.3) (end 161.29 115.57) (width 2) (layer "B.Cu") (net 1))
 (segment (start 78.74 87.63) (end 78.74 97.79) (width 2) (layer "B.Cu") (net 1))
 (segment (start 84.37 82) (end 78.74 87.63) (width 2) (layer "B.Cu") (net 1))
 (segment (start 111.3564 66.9064) (end 110.49 66.04) (width 1) (layer "B.Cu") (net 1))
 (segment (start 91.445 82) (end 91.44 81.995) (width 1) (layer "B.Cu") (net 1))
 (segment (start 104.14 91.44) (end 109.22 96.52) (width 1) (layer "B.Cu") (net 26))
 (segment (start 109.22 96.52) (end 109.22 99.06) (width 1) (layer "B.Cu") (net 26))
 (segment (start 109.22 99.06) (end 111.76 99.06) (width 1) (layer "B.Cu") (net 26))
 (segment (start 101.6 91.44) (end 104.14 91.44) (width 1) (layer "B.Cu") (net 26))
 (segment (start 101.6 88.9) (end 101.6 91.44) (width 1) (layer "B.Cu") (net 26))
 (segment (start 111.76 101.6) (end 106.68 101.6) (width 1) (layer "B.Cu") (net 27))
 (segment (start 106.68 96.52) (end 104.14 93.98) (width 1) (layer "B.Cu") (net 27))
 (segment (start 104.14 93.98) (end 99.06 93.98) (width 1) (layer "B.Cu") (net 27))
 (segment (start 106.68 101.6) (end 106.68 96.52) (width 1) (layer "B.Cu") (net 27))
 (segment (start 99.06 93.98) (end 99.06 88.9) (width 1) (layer "B.Cu") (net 27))
 (segment (start 101.6 104.14) (end 111.76 104.14) (width 1) (layer "B.Cu") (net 19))
 (segment (start 101.6 109.22) (end 111.76 109.22) (width 1) (layer "B.Cu") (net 17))
 (segment (start 97 99.06) (end 97 109.22) (width 1) (layer "B.Cu") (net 17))
 (segment (start 97 109.22) (end 101.6 109.22) (width 1) (layer "B.Cu") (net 17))
 (segment (start 101.6 99.06) (end 97 99.06) (width 1) (layer "B.Cu") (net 17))
 (segment (start 99.06 106.68) (end 101.6 106.68) (width 1) (layer "B.Cu") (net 18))
 (segment (start 101.6 101.6) (end 99.06 101.6) (width 1) (layer "B.Cu") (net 18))
 (segment (start 101.6 106.68) (end 111.76 106.68) (width 1) (layer "B.Cu") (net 18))
 (segment (start 99.06 101.6) (end 99.06 106.68) (width 1) (layer "B.Cu") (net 18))
 (segment (start 157.48 110.49) (end 149.86 102.87) (width 1) (layer "F.Cu") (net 2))
 (segment (start 149.86 102.87) (end 149.86 93.98) (width 1) (layer "F.Cu") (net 2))
 (segment (start 96.52 118.11) (end 105.41 118.11) (width 1) (layer "F.Cu") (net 2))
 (segment (start 106.68 116.84) (end 106.68 115.57) (width 1) (layer "F.Cu") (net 2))
 (segment (start 157.48 111.76) (end 157.48 110.49) (width 1) (layer "F.Cu") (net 2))
 (segment (start 105.41 118.11) (end 106.68 116.84) (width 1) (layer "F.Cu") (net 2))
 (segment (start 82 100) (end 82.44 100.44) (width 1) (layer "F.Cu") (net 2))
 (segment (start 82 92.71) (end 82 100) (width 1) (layer "F.Cu") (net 2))
 (via (at 96.52 118.11) (size 2) (drill 0.8) (layers "F.Cu" "B.Cu") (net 2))
 (via (at 157.48 111.76) (size 2) (drill 0.8) (layers "F.Cu" "B.Cu") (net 2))
 (via (at 82.44 100.44) (size 2) (drill 0.8) (layers "F.Cu" "B.Cu") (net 2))
 (via (at 149.86 93.98) (size 2) (drill 0.8) (layers "F.Cu" "B.Cu") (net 2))
 (via (at 106.68 115.57) (size 2) (drill 0.8) (layers "F.Cu" "B.Cu") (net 2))
 (via (at 82 92.71) (size 2) (drill 0.8) (layers "F.Cu" "B.Cu") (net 2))
 (segment (start 95.89 87) (end 95.25 86.36) (width 1) (layer "B.Cu") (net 2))
 (segment (start 114.3 62.23) (end 115.57 63.5) (width 1) (layer "B.Cu") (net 2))
 (segment (start 85.09 120.65) (end 81.28 116.84) (width 1) (layer "B.Cu") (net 2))
 (segment (start 149.86 93.98) (end 149.86 88.9) (width 1) (layer "B.Cu") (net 2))
 (segment (start 157.48 113.03) (end 157.48 119.38) (width 1) (layer "B.Cu") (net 2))
 (segment (start 115.57 82.55) (end 114.555 83.565) (width 1) (layer "B.Cu") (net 2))
 (segment (start 83.82 99.06) (end 86.36 99.06) (width 1) (layer "B.Cu") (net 2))
 (segment (start 107.95 114.3) (end 106.68 115.57) (width 1) (layer "B.Cu") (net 2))
 (segment (start 111.3564 84.285) (end 111.3564 85.4936) (width 1) (layer "B.Cu") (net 2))
 (segment (start 156.21 120.65) (end 95.25 120.65) (width 1) (layer "B.Cu") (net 2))
 (segment (start 157.48 113.03) (end 157.48 111.76) (width 1) (layer "B.Cu") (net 2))
 (segment (start 95.25 120.65) (end 85.09 120.65) (width 1) (layer "B.Cu") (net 2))
 (segment (start 82 90) (end 85.64 86.36) (width 1) (layer "B.Cu") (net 2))
 (segment (start 112.0764 83.565) (end 111.3564 84.285) (width 1) (layer "B.Cu") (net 2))
 (segment (start 114.3 55.88) (end 114.3 62.23) (width 1) (layer "B.Cu") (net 2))
 (segment (start 111.76 114.3) (end 107.95 114.3) (width 1) (layer "B.Cu") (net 2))
 (segment (start 160.02 111.76) (end 158.75 111.76) (width 1) (layer "B.Cu") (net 2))
 (segment (start 81.28 116.84) (end 81.28 101.6) (width 1) (layer "B.Cu") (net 2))
 (segment (start 96.52 119.38) (end 96.52 118.11) (width 1) (layer "B.Cu") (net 2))
 (segment (start 95.25 120.65) (end 96.52 119.38) (width 1) (layer "B.Cu") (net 2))
 (segment (start 81.28 101.6) (end 83.82 99.06) (width 1) (layer "B.Cu") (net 2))
 (segment (start 85.64 86.36) (end 95.25 86.36) (width 1) (layer "B.Cu") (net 2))
 (segment (start 114.555 83.565) (end 112.0764 83.565) (width 1) (layer "B.Cu") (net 2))
 (segment (start 111.3564 85.4936) (end 109.85 87) (width 1) (layer "B.Cu") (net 2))
 (segment (start 96.52 87.63) (end 95.25 86.36) (width 1) (layer "B.Cu") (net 2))
 (segment (start 157.48 119.38) (end 156.21 120.65) (width 1) (layer "B.Cu") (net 2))
 (segment (start 81.28 101.6) (end 82.44 100.44) (width 1) (layer "B.Cu") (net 2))
 (segment (start 82 92.71) (end 82 90) (width 1) (layer "B.Cu") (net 2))
 (segment (start 158.75 111.76) (end 157.48 113.03) (width 1) (layer "B.Cu") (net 2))
 (segment (start 115.57 63.5) (end 115.57 82.55) (width 1) (layer "B.Cu") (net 2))
 (segment (start 109.85 87) (end 95.89 87) (width 1) (layer "B.Cu") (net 2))
 (segment (start 96.52 88.9) (end 96.52 87.63) (width 1) (layer "B.Cu") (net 2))
 (segment (start 137.16 109.22) (end 142.24 114.3) (width 1) (layer "B.Cu") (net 6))
 (segment (start 152.4 114.3) (end 152.4 99.06) (width 1) (layer "B.Cu") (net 6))
 (segment (start 152.4 99.06) (end 144.78 99.06) (width 1) (layer "B.Cu") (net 6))
 (segment (start 144.78 114.3) (end 152.4 114.3) (width 1) (layer "B.Cu") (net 6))
 (segment (start 142.24 114.3) (end 144.78 114.3) (width 1) (layer "B.Cu") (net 6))
 (segment (start 134.62 109.22) (end 137.16 109.22) (width 1) (layer "B.Cu") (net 6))
 (segment (start 142.24 109.22) (end 137.16 104.14) (width 1) (layer "B.Cu") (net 8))
 (segment (start 137.16 104.14) (end 134.62 104.14) (width 1) (layer "B.Cu") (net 8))
 (segment (start 147.32 109.22) (end 144.78 109.22) (width 1) (layer "B.Cu") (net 8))
 (segment (start 144.78 104.14) (end 147.32 104.14) (width 1) (layer "B.Cu") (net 8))
 (segment (start 144.78 109.22) (end 142.24 109.22) (width 1) (layer "B.Cu") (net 8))
 (segment (start 147.32 104.14) (end 147.32 109.22) (width 1) (layer "B.Cu") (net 8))
 (segment (start 142.24 111.76) (end 137.16 106.68) (width 1) (layer "B.Cu") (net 7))
 (segment (start 144.78 101.6) (end 149.86 101.6) (width 1) (layer "B.Cu") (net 7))
 (segment (start 149.86 101.6) (end 149.86 111.76) (width 1) (layer "B.Cu") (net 7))
 (segment (start 137.16 106.68) (end 134.62 106.68) (width 1) (layer "B.Cu") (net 7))
 (segment (start 149.86 111.76) (end 144.78 111.76) (width 1) (layer "B.Cu") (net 7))
 (segment (start 144.78 111.76) (end 142.24 111.76) (width 1) (layer "B.Cu") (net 7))
 (segment (start 144.78 106.68) (end 142.24 106.68) (width 1) (layer "B.Cu") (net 9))
 (segment (start 142.24 106.68) (end 137.16 101.6) (width 1) (layer "B.Cu") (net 9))
 (segment (start 137.16 101.6) (end 134.62 101.6) (width 1) (layer "B.Cu") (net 9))
 (segment (start 147.32 91.44) (end 147.32 88.9) (width 1) (layer "B.Cu") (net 12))
 (segment (start 139.7 99.06) (end 139.7 96.52) (width 1) (layer "B.Cu") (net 12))
 (segment (start 134.62 99.06) (end 139.7 99.06) (width 1) (layer "B.Cu") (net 12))
 (segment (start 144.78 93.98) (end 147.32 91.44) (width 1) (layer "B.Cu") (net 12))
 (segment (start 142.24 93.98) (end 144.78 93.98) (width 1) (layer "B.Cu") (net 12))
 (segment (start 139.7 96.52) (end 142.24 93.98) (width 1) (layer "B.Cu") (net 12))
 (segment (start 139.7 91.44) (end 134.62 96.52) (width 1) (layer "B.Cu") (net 11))
 (segment (start 144.78 88.9) (end 144.78 91.44) (width 1) (layer "B.Cu") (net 11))
 (segment (start 144.78 91.44) (end 139.7 91.44) (width 1) (layer "B.Cu") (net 11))
 (segment (start 119.38 57.15) (end 119.38 55.88) (width 1) (layer "B.Cu") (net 24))
 (segment (start 118.11 96.52) (end 118.11 58.42) (width 1) (layer "B.Cu") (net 24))
 (segment (start 118.11 58.42) (end 119.38 57.15) (width 1) (layer "B.Cu") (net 24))
 (segment (start 115.57 99.06) (end 118.11 96.52) (width 1) (layer "B.Cu") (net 24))
 (segment (start 114.3 99.06) (end 115.57 99.06) (width 1) (layer "B.Cu") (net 24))
 (segment (start 121.92 58.42) (end 121.92 55.88) (width 1) (layer "B.Cu") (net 23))
 (segment (start 120.65 97.79) (end 120.65 59.69) (width 1) (layer "B.Cu") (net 23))
 (segment (start 120.65 59.69) (end 121.92 58.42) (width 1) (layer "B.Cu") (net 23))
 (segment (start 114.3 101.6) (end 116.84 101.6) (width 1) (layer "B.Cu") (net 23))
 (segment (start 116.84 101.6) (end 120.65 97.79) (width 1) (layer "B.Cu") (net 23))
 (segment (start 124.46 59.69) (end 124.46 55.88) (width 1) (layer "B.Cu") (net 22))
 (segment (start 118.11 104.14) (end 123.19 99.06) (width 1) (layer "B.Cu") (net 22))
 (segment (start 123.19 60.96) (end 124.46 59.69) (width 1) (layer "B.Cu") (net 22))
 (segment (start 114.3 104.14) (end 118.11 104.14) (width 1) (layer "B.Cu") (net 22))
 (segment (start 123.19 99.06) (end 123.19 60.96) (width 1) (layer "B.Cu") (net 22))
 (segment (start 125.73 100.33) (end 125.73 62.23) (width 1) (layer "B.Cu") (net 21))
 (segment (start 119.38 106.68) (end 125.73 100.33) (width 1) (layer "B.Cu") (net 21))
 (segment (start 127 60.96) (end 127 55.88) (width 1) (layer "B.Cu") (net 21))
 (segment (start 114.3 106.68) (end 119.38 106.68) (width 1) (layer "B.Cu") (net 21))
 (segment (start 125.73 62.23) (end 127 60.96) (width 1) (layer "B.Cu") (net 21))
 (segment (start 128.27 101.6) (end 128.27 64.77) (width 1) (layer "B.Cu") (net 20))
 (segment (start 128.27 64.77) (end 129.54 63.5) (width 1) (layer "B.Cu") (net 20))
 (segment (start 114.3 109.22) (end 120.65 109.22) (width 1) (layer "B.Cu") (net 20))
 (segment (start 129.54 63.5) (end 129.54 55.88) (width 1) (layer "B.Cu") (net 20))
 (segment (start 120.65 109.22) (end 128.27 101.6) (width 1) (layer "B.Cu") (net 20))
 (segment (start 95 96.52) (end 95 111.76) (width 1) (layer "B.Cu") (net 16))
 (segment (start 101.6 96.52) (end 95 96.52) (width 1) (layer "B.Cu") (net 16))
 (segment (start 101.6 111.76) (end 111.76 111.76) (width 1) (layer "B.Cu") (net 16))
 (segment (start 95 111.76) (end 101.6 111.76) (width 1) (layer "B.Cu") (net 16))
 (segment (start 89 91.34) (end 91.44 88.9) (width 1.8) (layer "B.Cu") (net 14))
 (segment (start 86.36 104.14) (end 89 104.14) (width 1.8) (layer "B.Cu") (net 14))
 (segment (start 89 104.14) (end 89 91.34) (width 1.8) (layer "B.Cu") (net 14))
 (segment (start 83.82 104.14) (end 83.82 111.76) (width 1.5) (layer "B.Cu") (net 14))
 (segment (start 83.82 111.76) (end 86.36 111.76) (width 1.5) (layer "B.Cu") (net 14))
 (segment (start 86.36 104.14) (end 83.82 104.14) (width 1.5) (layer "B.Cu") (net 14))
 (segment (start 92 106.12) (end 92 93.42) (width 1.8) (layer "B.Cu") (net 15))
 (segment (start 92 93.42) (end 93.98 91.44) (width 1.8) (layer "B.Cu") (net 15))
 (segment (start 93.98 91.44) (end 93.98 88.9) (width 1.8) (layer "B.Cu") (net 15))
 (segment (start 88.9 109.22) (end 92 106.12) (width 1.8) (layer "B.Cu") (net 15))
 (segment (start 86.36 109.22) (end 88.9 109.22) (width 1.8) (layer "B.Cu") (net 15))
 (segment (start 86.36 106.68) (end 86.36 109.22) (width 1.5) (layer "B.Cu") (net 15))
 (segment (start 164 104) (end 164 99.06) (width 2) (layer "B.Cu") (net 4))
 (segment (start 162.56 99.06) (end 160.02 99.06) (width 2) (layer "B.Cu") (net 4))
 (segment (start 162.56 99.06) (end 164 99.06) (width 1) (layer "B.Cu") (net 4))
 (segment (start 160.02 106.68) (end 161.32 106.68) (width 2) (layer "B.Cu") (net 4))
 (segment (start 164 99.06) (end 164 94) (width 2) (layer "B.Cu") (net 4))
 (segment (start 161.32 106.68) (end 163 105) (width 2) (layer "B.Cu") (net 4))
 (segment (start 158.9 88.9) (end 154.94 88.9) (width 2) (layer "B.Cu") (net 4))
 (segment (start 163 105) (end 164 104) (width 2) (layer "B.Cu") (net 4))
 (segment (start 164 94) (end 158.9 88.9) (width 2) (layer "B.Cu") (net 4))
 (segment (start 152.4 91.4) (end 152.4 88.9) (width 2) (layer "B.Cu") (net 5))
 (segment (start 158 101.6) (end 156 99.6) (width 2) (layer "B.Cu") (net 5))
 (segment (start 160.02 101.6) (end 158 101.6) (width 2) (layer "B.Cu") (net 5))
 (segment (start 156 95) (end 152.4 91.4) (width 2) (layer "B.Cu") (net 5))
 (segment (start 156 99.6) (end 156 95) (width 2) (layer "B.Cu") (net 5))
 (segment (start 160.02 101.6) (end 160.02 104.14) (width 2) (layer "B.Cu") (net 5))
 (segment (start 100.33 69.85) (end 137.16 69.85) (width 1) (layer "F.Cu") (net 10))
 (via (at 137.16 69.85) (size 2) (drill 0.8) (layers "F.Cu" "B.Cu") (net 10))
 (via (at 100.33 69.85) (size 2) (drill 0.8) (layers "F.Cu" "B.Cu") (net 10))
 (segment (start 99.06 69.85) (end 100.33 69.85) (width 2) (layer "B.Cu") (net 10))
 (segment (start 144.82 73.7) (end 144.82 84) (width 2) (layer "B.Cu") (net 10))
 (segment (start 93.98 81.995) (end 93.98 74.93) (width 2) (layer "B.Cu") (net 10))
 (segment (start 140.97 69.85) (end 144.82 73.7) (width 2) (layer "B.Cu") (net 10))
 (segment (start 137.16 69.85) (end 140.97 69.85) (width 2) (layer "B.Cu") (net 10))
 (segment (start 93.98 74.93) (end 99.06 69.85) (width 2) (layer "B.Cu") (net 10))
 (segment (start 93.985 82) (end 93.98 81.995) (width 2) (layer "B.Cu") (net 10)))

